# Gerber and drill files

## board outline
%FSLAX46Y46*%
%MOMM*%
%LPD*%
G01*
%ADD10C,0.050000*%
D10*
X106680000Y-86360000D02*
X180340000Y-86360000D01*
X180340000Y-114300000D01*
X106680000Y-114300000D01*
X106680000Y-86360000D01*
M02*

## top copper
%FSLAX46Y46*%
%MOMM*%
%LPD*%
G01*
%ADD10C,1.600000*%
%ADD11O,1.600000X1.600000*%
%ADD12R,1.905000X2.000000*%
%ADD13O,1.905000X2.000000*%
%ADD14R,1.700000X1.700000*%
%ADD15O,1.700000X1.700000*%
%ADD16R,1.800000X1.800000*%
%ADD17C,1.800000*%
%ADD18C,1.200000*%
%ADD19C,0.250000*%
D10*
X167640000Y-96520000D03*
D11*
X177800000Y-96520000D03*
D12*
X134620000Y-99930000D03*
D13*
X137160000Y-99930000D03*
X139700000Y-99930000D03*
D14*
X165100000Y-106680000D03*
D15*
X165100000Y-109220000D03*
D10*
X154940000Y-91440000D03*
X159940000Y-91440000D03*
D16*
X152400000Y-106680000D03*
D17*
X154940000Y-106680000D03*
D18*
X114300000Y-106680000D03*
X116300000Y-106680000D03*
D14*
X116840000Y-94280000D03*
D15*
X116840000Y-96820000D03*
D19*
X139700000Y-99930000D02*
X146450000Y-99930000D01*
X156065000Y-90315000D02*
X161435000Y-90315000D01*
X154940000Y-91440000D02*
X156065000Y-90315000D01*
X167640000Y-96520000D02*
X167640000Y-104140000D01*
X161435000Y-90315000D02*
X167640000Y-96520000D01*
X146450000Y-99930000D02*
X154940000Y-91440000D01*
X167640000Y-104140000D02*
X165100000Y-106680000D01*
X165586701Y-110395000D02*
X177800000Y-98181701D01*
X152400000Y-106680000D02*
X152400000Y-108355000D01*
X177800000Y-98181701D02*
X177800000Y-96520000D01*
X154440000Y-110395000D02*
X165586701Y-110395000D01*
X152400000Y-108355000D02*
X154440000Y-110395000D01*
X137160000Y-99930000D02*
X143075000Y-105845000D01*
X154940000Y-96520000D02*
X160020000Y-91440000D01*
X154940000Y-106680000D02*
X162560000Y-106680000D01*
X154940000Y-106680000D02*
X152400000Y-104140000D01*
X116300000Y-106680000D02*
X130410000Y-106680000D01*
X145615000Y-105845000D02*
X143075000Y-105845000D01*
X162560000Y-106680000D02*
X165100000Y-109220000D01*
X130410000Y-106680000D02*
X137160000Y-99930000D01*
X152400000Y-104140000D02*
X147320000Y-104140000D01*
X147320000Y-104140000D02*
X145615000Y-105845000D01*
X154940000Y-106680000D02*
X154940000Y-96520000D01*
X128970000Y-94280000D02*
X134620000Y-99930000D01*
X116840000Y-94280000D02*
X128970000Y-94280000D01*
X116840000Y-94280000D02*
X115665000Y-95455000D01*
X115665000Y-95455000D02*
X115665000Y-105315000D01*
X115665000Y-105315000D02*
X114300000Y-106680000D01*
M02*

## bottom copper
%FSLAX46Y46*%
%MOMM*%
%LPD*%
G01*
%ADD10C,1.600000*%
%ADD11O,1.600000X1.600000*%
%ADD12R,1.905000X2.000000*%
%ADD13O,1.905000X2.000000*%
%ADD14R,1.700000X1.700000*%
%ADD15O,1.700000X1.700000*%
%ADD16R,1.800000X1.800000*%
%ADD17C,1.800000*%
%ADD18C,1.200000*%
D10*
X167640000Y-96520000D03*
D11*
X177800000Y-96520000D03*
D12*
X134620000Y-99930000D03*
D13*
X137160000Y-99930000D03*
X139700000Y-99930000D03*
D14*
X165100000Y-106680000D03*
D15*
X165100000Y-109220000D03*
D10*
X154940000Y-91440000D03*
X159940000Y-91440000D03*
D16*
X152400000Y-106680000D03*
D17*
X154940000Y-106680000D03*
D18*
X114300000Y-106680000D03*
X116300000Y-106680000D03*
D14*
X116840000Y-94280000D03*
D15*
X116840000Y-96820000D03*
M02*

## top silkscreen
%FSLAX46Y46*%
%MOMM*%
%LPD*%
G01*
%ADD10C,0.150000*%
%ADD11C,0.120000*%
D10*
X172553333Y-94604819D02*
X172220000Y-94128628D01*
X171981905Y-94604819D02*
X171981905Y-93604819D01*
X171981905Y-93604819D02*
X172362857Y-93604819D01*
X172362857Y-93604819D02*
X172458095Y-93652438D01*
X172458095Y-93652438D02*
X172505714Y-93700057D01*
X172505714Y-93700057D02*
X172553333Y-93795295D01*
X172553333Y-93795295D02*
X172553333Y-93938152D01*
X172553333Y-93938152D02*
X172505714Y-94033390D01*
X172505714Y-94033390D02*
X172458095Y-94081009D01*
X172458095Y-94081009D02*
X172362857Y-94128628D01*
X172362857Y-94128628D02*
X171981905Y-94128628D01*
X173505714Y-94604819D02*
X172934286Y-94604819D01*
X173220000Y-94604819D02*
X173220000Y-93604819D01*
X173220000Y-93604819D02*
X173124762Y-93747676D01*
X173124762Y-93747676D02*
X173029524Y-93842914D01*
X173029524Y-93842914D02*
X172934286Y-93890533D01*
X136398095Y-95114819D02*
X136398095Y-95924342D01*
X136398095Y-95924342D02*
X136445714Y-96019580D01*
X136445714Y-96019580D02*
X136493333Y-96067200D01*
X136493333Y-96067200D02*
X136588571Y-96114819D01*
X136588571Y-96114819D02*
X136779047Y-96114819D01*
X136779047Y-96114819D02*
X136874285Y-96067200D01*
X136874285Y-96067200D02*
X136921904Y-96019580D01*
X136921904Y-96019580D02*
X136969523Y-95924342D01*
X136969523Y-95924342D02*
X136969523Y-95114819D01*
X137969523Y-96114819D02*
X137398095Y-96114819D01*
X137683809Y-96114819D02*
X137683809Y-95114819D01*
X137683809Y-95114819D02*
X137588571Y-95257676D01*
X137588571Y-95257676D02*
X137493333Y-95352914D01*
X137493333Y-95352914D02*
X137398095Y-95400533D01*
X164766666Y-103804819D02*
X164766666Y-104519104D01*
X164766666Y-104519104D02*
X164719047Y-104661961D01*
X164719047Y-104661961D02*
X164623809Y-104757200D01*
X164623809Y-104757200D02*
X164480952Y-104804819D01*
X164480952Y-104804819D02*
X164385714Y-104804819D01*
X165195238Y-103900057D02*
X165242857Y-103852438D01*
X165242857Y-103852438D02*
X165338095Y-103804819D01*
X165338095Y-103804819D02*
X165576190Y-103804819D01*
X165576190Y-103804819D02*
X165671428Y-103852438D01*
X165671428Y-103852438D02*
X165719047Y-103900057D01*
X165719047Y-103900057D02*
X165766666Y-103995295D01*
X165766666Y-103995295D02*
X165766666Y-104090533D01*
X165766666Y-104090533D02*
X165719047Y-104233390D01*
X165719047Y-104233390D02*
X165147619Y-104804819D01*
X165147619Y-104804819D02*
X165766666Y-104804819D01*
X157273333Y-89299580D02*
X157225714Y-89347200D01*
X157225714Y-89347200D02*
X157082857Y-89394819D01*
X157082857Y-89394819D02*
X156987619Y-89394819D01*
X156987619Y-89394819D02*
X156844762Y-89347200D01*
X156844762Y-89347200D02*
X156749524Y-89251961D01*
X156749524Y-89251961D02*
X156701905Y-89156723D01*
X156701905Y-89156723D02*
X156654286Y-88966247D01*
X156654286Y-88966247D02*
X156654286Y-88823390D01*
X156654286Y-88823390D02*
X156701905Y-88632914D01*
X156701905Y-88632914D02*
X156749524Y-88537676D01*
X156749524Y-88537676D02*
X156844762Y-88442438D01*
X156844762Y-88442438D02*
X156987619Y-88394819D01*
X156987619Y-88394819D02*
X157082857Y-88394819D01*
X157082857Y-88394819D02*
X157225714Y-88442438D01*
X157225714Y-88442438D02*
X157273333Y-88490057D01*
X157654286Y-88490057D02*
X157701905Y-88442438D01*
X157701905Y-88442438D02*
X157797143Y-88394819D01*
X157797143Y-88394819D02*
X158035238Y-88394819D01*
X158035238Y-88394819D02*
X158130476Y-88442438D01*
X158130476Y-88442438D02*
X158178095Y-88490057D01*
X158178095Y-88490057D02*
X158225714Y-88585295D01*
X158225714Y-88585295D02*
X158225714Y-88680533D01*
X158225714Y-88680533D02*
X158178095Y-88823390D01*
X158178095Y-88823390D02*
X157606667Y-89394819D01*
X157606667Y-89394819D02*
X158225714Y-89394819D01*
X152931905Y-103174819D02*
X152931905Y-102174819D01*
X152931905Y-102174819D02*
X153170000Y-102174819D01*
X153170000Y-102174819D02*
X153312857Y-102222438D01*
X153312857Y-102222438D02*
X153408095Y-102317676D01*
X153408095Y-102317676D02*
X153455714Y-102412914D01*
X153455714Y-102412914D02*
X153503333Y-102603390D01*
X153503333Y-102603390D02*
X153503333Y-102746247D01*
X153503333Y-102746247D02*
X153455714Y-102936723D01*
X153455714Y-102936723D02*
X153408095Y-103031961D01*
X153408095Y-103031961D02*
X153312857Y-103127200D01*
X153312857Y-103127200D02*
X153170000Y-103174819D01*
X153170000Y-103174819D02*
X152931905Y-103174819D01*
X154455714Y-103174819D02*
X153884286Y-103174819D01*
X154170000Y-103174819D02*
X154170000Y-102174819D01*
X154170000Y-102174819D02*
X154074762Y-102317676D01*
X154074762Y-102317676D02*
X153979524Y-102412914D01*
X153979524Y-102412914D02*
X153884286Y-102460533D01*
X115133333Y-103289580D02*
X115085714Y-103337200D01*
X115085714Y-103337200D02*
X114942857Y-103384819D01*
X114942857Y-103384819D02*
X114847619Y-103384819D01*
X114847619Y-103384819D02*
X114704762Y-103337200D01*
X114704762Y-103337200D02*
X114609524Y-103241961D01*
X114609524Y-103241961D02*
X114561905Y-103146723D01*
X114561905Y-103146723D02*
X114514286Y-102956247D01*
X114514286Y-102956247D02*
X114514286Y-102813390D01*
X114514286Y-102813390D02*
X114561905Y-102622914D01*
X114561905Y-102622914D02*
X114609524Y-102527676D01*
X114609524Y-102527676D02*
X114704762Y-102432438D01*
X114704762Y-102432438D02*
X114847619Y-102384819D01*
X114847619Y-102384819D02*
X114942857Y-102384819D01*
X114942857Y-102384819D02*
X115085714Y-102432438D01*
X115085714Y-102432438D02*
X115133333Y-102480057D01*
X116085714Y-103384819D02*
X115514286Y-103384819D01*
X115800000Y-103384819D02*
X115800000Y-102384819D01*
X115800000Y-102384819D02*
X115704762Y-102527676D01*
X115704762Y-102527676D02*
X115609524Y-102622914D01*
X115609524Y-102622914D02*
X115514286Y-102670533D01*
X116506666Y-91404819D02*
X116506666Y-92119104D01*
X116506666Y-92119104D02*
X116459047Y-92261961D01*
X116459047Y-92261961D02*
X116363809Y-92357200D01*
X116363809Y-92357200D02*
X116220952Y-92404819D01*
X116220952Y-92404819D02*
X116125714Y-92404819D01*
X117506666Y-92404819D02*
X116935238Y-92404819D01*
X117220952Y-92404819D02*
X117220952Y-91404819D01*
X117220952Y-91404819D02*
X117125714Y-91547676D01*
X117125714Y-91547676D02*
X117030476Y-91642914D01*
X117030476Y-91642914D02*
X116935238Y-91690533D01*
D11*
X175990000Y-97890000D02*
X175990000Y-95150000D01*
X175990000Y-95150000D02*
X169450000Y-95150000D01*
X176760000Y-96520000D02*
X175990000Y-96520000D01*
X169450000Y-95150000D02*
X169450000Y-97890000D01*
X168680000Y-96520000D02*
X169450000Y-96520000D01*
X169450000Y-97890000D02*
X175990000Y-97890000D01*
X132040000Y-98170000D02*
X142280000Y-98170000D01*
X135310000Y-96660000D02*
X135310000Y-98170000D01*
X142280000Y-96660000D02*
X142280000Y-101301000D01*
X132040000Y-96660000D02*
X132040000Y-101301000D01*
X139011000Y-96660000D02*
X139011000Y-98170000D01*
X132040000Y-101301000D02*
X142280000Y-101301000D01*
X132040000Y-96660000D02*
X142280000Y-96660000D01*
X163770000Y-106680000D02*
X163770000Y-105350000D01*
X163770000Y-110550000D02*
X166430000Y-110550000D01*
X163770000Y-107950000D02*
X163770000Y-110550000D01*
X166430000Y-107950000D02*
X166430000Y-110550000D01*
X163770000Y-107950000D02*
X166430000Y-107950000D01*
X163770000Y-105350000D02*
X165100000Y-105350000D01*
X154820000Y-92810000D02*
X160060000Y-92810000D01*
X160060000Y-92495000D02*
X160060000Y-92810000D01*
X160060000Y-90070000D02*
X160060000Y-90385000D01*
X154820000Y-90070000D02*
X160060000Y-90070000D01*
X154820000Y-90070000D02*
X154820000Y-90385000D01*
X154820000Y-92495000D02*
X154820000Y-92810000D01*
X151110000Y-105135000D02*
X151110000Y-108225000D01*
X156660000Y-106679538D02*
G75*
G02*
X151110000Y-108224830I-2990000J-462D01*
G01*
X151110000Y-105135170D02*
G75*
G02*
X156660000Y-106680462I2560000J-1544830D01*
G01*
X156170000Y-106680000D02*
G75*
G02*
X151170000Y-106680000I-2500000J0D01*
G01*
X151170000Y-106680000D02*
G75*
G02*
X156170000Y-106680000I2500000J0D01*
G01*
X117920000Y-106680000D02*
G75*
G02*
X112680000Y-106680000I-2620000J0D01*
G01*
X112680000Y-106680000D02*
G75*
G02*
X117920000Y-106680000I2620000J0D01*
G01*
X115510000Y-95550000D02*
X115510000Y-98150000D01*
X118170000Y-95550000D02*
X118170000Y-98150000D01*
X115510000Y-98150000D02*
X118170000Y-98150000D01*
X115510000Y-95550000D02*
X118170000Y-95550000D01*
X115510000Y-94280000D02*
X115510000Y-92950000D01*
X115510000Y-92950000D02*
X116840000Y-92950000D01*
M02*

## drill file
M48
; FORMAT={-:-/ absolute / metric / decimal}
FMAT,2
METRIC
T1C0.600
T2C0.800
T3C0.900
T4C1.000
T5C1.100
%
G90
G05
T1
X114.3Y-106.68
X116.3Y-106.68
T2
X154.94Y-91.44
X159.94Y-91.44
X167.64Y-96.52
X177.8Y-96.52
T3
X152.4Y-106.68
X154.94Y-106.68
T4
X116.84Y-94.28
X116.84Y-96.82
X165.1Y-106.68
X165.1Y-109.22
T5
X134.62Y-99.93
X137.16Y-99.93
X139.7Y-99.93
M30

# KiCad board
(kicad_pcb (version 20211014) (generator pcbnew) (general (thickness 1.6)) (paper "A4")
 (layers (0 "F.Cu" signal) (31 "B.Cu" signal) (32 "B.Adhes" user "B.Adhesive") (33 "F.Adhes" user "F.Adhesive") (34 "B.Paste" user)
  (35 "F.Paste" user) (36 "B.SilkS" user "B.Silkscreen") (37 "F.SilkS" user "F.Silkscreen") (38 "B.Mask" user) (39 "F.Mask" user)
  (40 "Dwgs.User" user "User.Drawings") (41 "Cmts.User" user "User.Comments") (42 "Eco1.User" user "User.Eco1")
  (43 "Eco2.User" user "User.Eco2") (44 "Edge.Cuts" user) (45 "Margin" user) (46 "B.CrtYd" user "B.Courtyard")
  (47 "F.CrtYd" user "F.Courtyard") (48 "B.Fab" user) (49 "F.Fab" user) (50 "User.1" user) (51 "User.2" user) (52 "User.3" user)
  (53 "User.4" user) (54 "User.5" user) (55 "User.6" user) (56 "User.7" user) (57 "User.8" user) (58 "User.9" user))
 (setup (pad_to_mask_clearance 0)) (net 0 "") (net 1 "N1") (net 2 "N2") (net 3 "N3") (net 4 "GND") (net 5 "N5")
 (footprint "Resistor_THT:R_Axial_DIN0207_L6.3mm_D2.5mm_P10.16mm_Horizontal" (layer "F.Cu") (at 167.64 96.52)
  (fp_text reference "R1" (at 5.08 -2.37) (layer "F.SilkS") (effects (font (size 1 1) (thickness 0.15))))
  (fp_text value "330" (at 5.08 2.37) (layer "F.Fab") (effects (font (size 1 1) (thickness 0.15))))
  (fp_line (start 8.35 1.37) (end 8.35 -1.37) (layer "F.SilkS") (width 0.12))
  (fp_line (start 8.35 -1.37) (end 1.81 -1.37) (layer "F.SilkS") (width 0.12))
  (fp_line (start 9.12 0) (end 8.35 0) (layer "F.SilkS") (width 0.12))
  (fp_line (start 1.81 -1.37) (end 1.81 1.37) (layer "F.SilkS") (width 0.12))
  (fp_line (start 1.04 0) (end 1.81 0) (layer "F.SilkS") (width 0.12))
  (fp_line (start 1.81 1.37) (end 8.35 1.37) (layer "F.SilkS") (width 0.12))
  (pad "1" thru_hole circle (at 0 0) (size 1.6 1.6) (drill 0.8) (layers *.Cu *.Mask) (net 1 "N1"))
  (pad "2" thru_hole oval (at 10.16 0) (size 1.6 1.6) (drill 0.8) (layers *.Cu *.Mask) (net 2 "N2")))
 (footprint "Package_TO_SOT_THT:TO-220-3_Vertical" (layer "F.Cu") (at 134.62 99.93)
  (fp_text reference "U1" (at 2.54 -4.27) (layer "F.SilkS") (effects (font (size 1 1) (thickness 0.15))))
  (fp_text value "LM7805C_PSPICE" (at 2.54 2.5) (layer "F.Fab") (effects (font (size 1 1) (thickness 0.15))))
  (fp_line (start -2.58 -1.76) (end 7.66 -1.76) (layer "F.SilkS") (width 0.12))
  (fp_line (start 0.69 -3.27) (end 0.69 -1.76) (layer "F.SilkS") (width 0.12))
  (fp_line (start 7.66 -3.27) (end 7.66 1.371) (layer "F.SilkS") (width 0.12))
  (fp_line (start -2.58 -3.27) (end -2.58 1.371) (layer "F.SilkS") (width 0.12))
  (fp_line (start 4.391 -3.27) (end 4.391 -1.76) (layer "F.SilkS") (width 0.12))
  (fp_line (start -2.58 1.371) (end 7.66 1.371) (layer "F.SilkS") (width 0.12))
  (fp_line (start -2.58 -3.27) (end 7.66 -3.27) (layer "F.SilkS") (width 0.12))
  (pad "1" thru_hole rect (at 0 0) (size 1.905 2) (drill 1.1) (layers *.Cu *.Mask) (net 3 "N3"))
  (pad "2" thru_hole oval (at 2.54 0) (size 1.905 2) (drill 1.1) (layers *.Cu *.Mask) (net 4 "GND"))
  (pad "3" thru_hole oval (at 5.08 0) (size 1.905 2) (drill 1.1) (layers *.Cu *.Mask) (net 1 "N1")))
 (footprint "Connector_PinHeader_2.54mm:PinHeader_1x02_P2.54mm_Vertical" (layer "F.Cu") (at 165.1 106.68)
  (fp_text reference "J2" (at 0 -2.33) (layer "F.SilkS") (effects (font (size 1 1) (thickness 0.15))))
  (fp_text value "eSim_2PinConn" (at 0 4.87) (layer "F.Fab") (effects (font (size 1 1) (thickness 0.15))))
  (fp_line (start -1.33 0) (end -1.33 -1.33) (layer "F.SilkS") (width 0.12))
  (fp_line (start -1.33 3.87) (end 1.33 3.87) (layer "F.SilkS") (width 0.12))
  (fp_line (start -1.33 1.27) (end -1.33 3.87) (layer "F.SilkS") (width 0.12))
  (fp_line (start 1.33 1.27) (end 1.33 3.87) (layer "F.SilkS") (width 0.12))
  (fp_line (start -1.33 1.27) (end 1.33 1.27) (layer "F.SilkS") (width 0.12))
  (fp_line (start -1.33 -1.33) (end 0 -1.33) (layer "F.SilkS") (width 0.12))
  (pad "1" thru_hole rect (at 0 0) (size 1.7 1.7) (drill 1) (layers *.Cu *.Mask) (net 1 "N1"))
  (pad "2" thru_hole oval (at 0 2.54) (size 1.7 1.7) (drill 1) (layers *.Cu *.Mask) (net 4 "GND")))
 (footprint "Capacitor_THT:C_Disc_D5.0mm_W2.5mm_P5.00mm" (layer "F.Cu") (at 154.94 91.44)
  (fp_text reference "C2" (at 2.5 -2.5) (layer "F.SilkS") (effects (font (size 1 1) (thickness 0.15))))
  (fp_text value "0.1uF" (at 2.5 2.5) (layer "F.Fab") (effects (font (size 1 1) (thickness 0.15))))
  (fp_line (start -0.12 1.37) (end 5.12 1.37) (layer "F.SilkS") (width 0.12))
  (fp_line (start 5.12 1.055) (end 5.12 1.37) (layer "F.SilkS") (width 0.12))
  (fp_line (start 5.12 -1.37) (end 5.12 -1.055) (layer "F.SilkS") (width 0.12))
  (fp_line (start -0.12 -1.37) (end 5.12 -1.37) (layer "F.SilkS") (width 0.12))
  (fp_line (start -0.12 -1.37) (end -0.12 -1.055) (layer "F.SilkS") (width 0.12))
  (fp_line (start -0.12 1.055) (end -0.12 1.37) (layer "F.SilkS") (width 0.12))
  (pad "1" thru_hole circle (at 0 0) (size 1.6 1.6) (drill 0.8) (layers *.Cu *.Mask) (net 1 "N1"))
  (pad "2" thru_hole circle (at 5 0) (size 1.6 1.6) (drill 0.8) (layers *.Cu *.Mask) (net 4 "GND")))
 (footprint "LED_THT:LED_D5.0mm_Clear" (layer "F.Cu") (at 152.4 106.68)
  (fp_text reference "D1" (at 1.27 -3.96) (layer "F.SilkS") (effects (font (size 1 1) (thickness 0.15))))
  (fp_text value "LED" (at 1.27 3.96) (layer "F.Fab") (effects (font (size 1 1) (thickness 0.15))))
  (fp_line (start -1.29 -1.545) (end -1.29 1.545) (layer "F.SilkS") (width 0.12))
  (fp_arc (start 4.26 -0.000462) (mid 2.072002 2.880433) (end -1.29 1.54483) (layer "F.SilkS") (width 0.12))
  (fp_arc (start -1.29 -1.54483) (mid 2.072002 -2.880433) (end 4.26 0.000462) (layer "F.SilkS") (width 0.12))
  (fp_circle (center 1.27 0) (end 3.77 0) (layer "F.SilkS") (width 0.12) (fill none))
  (pad "1" thru_hole rect (at 0 0) (size 1.8 1.8) (drill 0.9) (layers *.Cu *.Mask) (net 2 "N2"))
  (pad "2" thru_hole circle (at 2.54 0) (size 1.8 1.8) (drill 0.9) (layers *.Cu *.Mask) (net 4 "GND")))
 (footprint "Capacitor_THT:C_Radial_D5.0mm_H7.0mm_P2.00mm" (layer "F.Cu") (at 114.3 106.68)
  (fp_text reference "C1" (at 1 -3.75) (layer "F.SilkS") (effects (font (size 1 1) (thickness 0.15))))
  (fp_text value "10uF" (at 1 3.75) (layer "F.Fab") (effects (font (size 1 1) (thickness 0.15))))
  (fp_circle (center 1 0) (end 3.62 0) (layer "F.SilkS") (width 0.12) (fill none))
  (pad "1" thru_hole circle (at 0 0) (size 1.2 1.2) (drill 0.6) (layers *.Cu *.Mask) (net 3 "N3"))
  (pad "2" thru_hole circle (at 2 0) (size 1.2 1.2) (drill 0.6) (layers *.Cu *.Mask) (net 4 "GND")))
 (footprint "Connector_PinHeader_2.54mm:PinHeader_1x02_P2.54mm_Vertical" (layer "F.Cu") (at 116.84 94.28)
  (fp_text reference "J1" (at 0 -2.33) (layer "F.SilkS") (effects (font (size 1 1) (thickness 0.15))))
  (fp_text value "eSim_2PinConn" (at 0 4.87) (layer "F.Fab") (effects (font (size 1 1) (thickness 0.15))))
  (fp_line (start -1.33 1.27) (end -1.33 3.87) (layer "F.SilkS") (width 0.12))
  (fp_line (start 1.33 1.27) (end 1.33 3.87) (layer "F.SilkS") (width 0.12))
  (fp_line (start -1.33 3.87) (end 1.33 3.87) (layer "F.SilkS") (width 0.12))
  (fp_line (start -1.33 1.27) (end 1.33 1.27) (layer "F.SilkS") (width 0.12))
  (fp_line (start -1.33 0) (end -1.33 -1.33) (layer "F.SilkS") (width 0.12))
  (fp_line (start -1.33 -1.33) (end 0 -1.33) (layer "F.SilkS") (width 0.12))
  (pad "1" thru_hole rect (at 0 0) (size 1.7 1.7) (drill 1) (layers *.Cu *.Mask) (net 3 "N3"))
  (pad "2" thru_hole oval (at 0 2.54) (size 1.7 1.7) (drill 1) (layers *.Cu *.Mask) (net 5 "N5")))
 (gr_rect (start 106.68 86.36) (end 180.34 114.3) (layer "Edge.Cuts") (width 0.05) (fill none))
 (segment (start 139.7 99.93) (end 146.45 99.93) (width 0.25) (layer "F.Cu") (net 1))
 (segment (start 156.065 90.315) (end 161.435 90.315) (width 0.25) (layer "F.Cu") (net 1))
 (segment (start 154.94 91.44) (end 156.065 90.315) (width 0.25) (layer "F.Cu") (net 1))
 (segment (start 167.64 96.52) (end 167.64 104.14) (width 0.25) (layer "F.Cu") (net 1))
 (segment (start 161.435 90.315) (end 167.64 96.52) (width 0.25) (layer "F.Cu") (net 1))
 (segment (start 146.45 99.93) (end 154.94 91.44) (width 0.25) (layer "F.Cu") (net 1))
 (segment (start 167.64 104.14) (end 165.1 106.68) (width 0.25) (layer "F.Cu") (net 1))
 (segment (start 165.586701 110.395) (end 177.8 98.181701) (width 0.25) (layer "F.Cu") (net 2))
 (segment (start 152.4 106.68) (end 152.4 108.355) (width 0.25) (layer "F.Cu") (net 2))
 (segment (start 177.8 98.181701) (end 177.8 96.52) (width 0.25) (layer "F.Cu") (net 2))
 (segment (start 154.44 110.395) (end 165.586701 110.395) (width 0.25) (layer "F.Cu") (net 2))
 (segment (start 152.4 108.355) (end 154.44 110.395) (width 0.25) (layer "F.Cu") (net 2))
 (segment (start 137.16 99.93) (end 143.075 105.845) (width 0.25) (layer "F.Cu") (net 4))
 (segment (start 154.94 96.52) (end 160.02 91.44) (width 0.25) (layer "F.Cu") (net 4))
 (segment (start 154.94 106.68) (end 162.56 106.68) (width 0.25) (layer "F.Cu") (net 4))
 (segment (start 154.94 106.68) (end 152.4 104.14) (width 0.25) (layer "F.Cu") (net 4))
 (segment (start 116.3 106.68) (end 130.41 106.68) (width 0.25) (layer "F.Cu") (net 4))
 (segment (start 145.615 105.845) (end 143.075 105.845) (width 0.25) (layer "F.Cu") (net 4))
 (segment (start 162.56 106.68) (end 165.1 109.22) (width 0.25) (layer "F.Cu") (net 4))
 (segment (start 130.41 106.68) (end 137.16 99.93) (width 0.25) (layer "F.Cu") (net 4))
 (segment (start 152.4 104.14) (end 147.32 104.14) (width 0.25) (layer "F.Cu") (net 4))
 (segment (start 147.32 104.14) (end 145.615 105.845) (width 0.25) (layer "F.Cu") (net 4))
 (segment (start 154.94 106.68) (end 154.94 96.52) (width 0.25) (layer "F.Cu") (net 4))
 (segment (start 128.97 94.28) (end 134.62 99.93) (width 0.25) (layer "F.Cu") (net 3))
 (segment (start 116.84 94.28) (end 128.97 94.28) (width 0.25) (layer "F.Cu") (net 3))
 (segment (start 116.84 94.28) (end 115.665 95.455) (width 0.25) (layer "F.Cu") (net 3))
 (segment (start 115.665 95.455) (end 115.665 105.315) (width 0.25) (layer "F.Cu") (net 3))
 (segment (start 115.665 105.315) (end 114.3 106.68) (width 0.25) (layer "F.Cu") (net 3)))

